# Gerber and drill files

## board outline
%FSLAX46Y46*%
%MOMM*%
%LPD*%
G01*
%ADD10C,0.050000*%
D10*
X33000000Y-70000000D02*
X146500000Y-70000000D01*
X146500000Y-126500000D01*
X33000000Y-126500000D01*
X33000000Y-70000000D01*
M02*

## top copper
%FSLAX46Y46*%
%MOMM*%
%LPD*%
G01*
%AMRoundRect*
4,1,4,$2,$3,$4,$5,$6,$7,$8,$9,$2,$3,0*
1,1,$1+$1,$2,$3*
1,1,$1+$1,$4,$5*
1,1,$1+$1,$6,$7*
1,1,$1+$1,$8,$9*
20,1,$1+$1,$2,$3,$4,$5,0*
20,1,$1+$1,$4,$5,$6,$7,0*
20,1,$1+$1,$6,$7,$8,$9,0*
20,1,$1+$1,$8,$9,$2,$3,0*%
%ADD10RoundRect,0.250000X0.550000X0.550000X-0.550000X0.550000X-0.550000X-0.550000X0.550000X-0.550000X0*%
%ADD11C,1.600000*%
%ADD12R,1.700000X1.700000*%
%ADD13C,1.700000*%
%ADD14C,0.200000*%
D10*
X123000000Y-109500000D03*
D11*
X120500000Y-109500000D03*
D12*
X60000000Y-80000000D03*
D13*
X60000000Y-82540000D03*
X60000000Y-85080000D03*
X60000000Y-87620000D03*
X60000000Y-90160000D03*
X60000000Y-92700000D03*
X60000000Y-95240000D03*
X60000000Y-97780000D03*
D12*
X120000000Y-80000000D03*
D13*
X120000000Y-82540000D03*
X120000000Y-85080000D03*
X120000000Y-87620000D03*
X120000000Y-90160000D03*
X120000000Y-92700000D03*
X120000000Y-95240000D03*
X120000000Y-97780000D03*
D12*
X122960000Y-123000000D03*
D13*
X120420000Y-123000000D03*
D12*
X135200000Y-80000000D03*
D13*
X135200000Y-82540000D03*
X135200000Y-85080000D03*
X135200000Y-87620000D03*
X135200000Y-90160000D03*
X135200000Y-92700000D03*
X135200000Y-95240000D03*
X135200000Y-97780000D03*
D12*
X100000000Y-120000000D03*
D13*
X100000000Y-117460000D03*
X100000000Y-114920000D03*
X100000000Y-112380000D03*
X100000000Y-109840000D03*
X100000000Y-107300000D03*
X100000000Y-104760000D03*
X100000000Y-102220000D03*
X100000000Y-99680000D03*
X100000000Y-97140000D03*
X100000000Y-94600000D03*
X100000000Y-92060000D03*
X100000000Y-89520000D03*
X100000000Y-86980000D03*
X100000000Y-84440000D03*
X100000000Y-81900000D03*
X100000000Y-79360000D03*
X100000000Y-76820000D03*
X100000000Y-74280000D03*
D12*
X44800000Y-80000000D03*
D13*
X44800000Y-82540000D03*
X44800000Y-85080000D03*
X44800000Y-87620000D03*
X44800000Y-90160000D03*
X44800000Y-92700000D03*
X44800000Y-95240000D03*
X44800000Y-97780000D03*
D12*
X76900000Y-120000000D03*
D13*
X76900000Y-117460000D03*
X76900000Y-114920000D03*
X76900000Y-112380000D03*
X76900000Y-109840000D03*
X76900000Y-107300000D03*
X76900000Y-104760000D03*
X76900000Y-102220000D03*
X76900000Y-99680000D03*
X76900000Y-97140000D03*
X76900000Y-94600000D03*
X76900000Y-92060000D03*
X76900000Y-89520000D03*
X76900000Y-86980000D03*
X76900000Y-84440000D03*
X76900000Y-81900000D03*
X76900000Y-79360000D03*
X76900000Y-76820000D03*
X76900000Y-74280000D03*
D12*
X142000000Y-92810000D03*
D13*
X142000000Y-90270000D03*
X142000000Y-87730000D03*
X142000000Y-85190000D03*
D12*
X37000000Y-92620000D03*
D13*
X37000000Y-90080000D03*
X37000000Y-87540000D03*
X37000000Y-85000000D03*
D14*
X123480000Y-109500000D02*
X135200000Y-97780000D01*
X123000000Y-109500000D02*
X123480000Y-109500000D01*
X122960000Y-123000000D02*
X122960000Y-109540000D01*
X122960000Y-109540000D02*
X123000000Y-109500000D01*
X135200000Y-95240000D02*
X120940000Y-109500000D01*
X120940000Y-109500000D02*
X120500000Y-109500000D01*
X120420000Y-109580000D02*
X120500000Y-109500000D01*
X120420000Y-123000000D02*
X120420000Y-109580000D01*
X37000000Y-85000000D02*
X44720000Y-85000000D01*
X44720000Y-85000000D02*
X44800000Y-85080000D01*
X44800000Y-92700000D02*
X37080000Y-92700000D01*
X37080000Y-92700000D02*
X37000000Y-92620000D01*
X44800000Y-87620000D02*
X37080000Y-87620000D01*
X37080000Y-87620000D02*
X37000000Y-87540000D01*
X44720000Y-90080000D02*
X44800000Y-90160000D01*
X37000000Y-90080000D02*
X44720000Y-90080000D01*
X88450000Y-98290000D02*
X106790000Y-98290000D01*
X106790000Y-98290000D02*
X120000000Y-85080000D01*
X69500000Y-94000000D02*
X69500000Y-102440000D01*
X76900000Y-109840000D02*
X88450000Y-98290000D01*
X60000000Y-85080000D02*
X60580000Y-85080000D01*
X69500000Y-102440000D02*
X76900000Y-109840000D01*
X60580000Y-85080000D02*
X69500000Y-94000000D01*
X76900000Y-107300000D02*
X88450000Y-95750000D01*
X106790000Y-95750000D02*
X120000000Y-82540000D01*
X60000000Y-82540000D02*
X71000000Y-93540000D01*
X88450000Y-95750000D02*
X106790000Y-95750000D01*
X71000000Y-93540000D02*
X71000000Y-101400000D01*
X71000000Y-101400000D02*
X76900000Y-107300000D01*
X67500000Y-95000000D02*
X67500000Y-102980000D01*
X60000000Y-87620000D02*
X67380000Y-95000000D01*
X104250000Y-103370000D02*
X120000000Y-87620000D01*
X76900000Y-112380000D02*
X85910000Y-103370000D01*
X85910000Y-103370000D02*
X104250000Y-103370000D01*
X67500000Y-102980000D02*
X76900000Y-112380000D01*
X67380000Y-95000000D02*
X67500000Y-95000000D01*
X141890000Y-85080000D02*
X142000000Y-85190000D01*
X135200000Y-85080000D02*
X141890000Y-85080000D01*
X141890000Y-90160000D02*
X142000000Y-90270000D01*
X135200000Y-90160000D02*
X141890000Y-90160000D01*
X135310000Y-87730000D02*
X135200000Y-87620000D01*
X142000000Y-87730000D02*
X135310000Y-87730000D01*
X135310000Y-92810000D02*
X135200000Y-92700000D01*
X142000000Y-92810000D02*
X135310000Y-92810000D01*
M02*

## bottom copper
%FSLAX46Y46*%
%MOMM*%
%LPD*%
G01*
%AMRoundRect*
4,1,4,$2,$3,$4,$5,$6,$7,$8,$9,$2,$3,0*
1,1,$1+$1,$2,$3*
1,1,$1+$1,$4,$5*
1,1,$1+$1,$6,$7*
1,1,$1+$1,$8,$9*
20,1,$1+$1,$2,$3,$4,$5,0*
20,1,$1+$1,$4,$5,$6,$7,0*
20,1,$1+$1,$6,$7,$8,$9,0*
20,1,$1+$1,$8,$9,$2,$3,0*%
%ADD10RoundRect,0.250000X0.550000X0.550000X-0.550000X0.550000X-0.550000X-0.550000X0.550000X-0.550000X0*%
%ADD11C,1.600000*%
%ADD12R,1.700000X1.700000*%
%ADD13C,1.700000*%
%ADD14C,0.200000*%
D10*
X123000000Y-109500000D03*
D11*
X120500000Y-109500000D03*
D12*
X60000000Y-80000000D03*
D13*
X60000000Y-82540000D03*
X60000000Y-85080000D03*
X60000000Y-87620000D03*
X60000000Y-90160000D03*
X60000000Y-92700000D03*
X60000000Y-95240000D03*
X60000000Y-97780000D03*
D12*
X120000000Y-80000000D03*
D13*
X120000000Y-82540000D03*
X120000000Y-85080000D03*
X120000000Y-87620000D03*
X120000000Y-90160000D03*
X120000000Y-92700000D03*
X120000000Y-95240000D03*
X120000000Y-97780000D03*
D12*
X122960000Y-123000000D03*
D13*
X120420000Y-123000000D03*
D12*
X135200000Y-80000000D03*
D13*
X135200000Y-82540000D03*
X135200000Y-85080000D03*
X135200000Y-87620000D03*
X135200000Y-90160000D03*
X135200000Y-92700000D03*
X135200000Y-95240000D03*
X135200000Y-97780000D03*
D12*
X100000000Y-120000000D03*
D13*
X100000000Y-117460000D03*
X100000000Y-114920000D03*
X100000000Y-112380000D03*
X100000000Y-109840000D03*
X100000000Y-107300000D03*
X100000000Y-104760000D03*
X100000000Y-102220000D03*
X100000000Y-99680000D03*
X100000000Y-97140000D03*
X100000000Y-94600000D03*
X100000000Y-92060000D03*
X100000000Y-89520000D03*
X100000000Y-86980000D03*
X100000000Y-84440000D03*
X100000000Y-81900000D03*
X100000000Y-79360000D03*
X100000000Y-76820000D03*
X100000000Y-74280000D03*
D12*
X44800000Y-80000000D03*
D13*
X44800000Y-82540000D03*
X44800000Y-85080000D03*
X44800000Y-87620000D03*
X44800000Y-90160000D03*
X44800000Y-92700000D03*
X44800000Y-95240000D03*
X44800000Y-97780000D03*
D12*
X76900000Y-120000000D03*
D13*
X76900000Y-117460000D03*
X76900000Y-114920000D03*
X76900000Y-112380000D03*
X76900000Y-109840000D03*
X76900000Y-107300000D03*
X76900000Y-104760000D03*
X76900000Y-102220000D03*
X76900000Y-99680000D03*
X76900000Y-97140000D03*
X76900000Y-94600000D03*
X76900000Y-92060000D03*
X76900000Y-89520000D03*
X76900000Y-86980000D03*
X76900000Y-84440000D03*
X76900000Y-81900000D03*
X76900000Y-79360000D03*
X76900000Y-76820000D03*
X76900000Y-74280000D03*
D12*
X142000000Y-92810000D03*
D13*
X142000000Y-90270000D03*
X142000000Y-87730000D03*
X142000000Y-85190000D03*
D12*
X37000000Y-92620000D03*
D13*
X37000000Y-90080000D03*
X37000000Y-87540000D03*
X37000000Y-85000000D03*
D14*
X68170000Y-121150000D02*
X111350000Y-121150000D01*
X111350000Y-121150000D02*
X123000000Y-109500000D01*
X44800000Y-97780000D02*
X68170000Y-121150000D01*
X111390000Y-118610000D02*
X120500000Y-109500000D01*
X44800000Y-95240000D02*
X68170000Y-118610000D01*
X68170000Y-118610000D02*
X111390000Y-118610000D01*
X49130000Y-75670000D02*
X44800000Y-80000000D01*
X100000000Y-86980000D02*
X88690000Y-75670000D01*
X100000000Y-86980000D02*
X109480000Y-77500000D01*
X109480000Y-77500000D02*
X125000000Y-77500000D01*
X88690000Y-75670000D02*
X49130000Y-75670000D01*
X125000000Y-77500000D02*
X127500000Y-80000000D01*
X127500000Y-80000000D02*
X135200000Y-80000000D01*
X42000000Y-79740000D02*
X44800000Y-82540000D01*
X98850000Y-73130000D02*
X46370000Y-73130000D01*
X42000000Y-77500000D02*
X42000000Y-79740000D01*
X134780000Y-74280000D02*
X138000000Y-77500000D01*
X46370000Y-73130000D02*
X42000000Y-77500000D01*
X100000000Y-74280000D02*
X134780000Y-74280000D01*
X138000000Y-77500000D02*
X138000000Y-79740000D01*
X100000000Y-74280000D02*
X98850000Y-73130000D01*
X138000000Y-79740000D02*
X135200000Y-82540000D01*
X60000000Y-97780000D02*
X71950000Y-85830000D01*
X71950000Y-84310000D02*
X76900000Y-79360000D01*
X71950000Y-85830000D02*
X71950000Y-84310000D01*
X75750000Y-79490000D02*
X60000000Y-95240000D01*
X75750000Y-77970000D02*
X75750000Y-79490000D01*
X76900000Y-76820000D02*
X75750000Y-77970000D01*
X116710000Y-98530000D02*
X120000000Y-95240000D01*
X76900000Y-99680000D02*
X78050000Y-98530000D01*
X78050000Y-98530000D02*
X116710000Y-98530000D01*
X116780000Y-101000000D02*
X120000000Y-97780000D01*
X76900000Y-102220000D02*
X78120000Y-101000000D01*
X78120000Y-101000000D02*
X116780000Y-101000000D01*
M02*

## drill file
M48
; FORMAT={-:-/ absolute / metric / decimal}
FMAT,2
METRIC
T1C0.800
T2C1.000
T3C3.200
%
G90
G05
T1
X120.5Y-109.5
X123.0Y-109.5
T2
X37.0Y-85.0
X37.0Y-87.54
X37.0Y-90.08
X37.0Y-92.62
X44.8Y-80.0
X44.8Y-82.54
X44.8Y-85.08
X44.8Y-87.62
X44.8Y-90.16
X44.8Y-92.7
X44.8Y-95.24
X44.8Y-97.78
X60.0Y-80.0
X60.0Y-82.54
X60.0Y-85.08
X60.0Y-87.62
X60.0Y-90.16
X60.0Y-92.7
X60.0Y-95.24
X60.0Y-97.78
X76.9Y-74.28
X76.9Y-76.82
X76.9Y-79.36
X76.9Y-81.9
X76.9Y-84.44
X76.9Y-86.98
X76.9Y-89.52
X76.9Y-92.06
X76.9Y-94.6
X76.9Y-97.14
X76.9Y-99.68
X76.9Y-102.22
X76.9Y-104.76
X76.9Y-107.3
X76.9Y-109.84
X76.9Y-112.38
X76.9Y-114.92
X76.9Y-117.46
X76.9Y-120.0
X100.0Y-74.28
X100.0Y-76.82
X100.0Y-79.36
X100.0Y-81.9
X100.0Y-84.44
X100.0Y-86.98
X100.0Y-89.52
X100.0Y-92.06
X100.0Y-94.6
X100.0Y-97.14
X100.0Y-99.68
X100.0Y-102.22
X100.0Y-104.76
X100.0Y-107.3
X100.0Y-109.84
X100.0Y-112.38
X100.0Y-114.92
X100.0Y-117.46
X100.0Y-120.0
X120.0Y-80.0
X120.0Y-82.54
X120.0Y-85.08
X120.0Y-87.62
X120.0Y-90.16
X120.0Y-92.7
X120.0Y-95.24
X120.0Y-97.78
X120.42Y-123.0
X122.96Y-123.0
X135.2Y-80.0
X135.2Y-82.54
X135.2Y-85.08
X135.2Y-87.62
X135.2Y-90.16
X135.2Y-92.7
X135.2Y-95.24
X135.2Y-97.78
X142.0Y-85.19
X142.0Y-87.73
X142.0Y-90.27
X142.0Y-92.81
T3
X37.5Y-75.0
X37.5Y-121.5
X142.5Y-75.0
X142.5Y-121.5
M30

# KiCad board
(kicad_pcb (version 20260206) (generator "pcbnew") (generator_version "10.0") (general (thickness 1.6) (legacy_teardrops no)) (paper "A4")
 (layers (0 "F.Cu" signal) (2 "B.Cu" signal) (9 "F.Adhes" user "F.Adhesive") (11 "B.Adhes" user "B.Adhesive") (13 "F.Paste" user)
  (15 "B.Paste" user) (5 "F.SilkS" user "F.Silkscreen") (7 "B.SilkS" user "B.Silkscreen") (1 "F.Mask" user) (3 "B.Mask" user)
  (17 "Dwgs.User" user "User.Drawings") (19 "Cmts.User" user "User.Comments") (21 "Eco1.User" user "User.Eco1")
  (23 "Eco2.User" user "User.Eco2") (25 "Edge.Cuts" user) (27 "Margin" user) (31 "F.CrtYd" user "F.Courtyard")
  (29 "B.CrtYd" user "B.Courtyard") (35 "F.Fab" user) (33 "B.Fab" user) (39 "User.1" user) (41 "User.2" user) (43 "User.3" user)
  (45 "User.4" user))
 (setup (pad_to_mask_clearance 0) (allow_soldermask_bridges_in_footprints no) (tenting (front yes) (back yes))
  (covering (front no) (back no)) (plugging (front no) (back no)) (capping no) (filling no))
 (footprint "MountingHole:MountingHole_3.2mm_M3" (layer "F.Cu") (at 37.5 121.5)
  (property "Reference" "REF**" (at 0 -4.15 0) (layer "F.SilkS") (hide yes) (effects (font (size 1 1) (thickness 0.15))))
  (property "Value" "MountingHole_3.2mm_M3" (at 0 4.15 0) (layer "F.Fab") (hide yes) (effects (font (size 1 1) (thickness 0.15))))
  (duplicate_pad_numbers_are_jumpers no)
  (pad "" np_thru_hole circle (at 0 0) (size 3.2 3.2) (drill 3.2) (layers "*.Cu" "*.Mask")))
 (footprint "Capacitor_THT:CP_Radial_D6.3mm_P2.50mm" (layer "F.Cu") (at 123 109.5 180)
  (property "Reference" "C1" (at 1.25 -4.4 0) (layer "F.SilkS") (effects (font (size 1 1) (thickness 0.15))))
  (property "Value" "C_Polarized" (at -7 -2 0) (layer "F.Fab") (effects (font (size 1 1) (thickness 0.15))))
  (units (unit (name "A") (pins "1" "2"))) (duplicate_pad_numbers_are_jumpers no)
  (pad "1" thru_hole roundrect (at 0 0 180) (size 1.6 1.6) (drill 0.8) (layers "*.Cu" "*.Mask") (remove_unused_layers no)
   (roundrect_rratio 0.15625) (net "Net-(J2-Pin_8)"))
  (pad "2" thru_hole circle (at 2.5 0 180) (size 1.6 1.6) (drill 0.8) (layers "*.Cu" "*.Mask") (remove_unused_layers no)
   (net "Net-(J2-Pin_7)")))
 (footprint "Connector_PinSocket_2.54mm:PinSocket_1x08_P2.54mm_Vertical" (layer "F.Cu") (at 60 80)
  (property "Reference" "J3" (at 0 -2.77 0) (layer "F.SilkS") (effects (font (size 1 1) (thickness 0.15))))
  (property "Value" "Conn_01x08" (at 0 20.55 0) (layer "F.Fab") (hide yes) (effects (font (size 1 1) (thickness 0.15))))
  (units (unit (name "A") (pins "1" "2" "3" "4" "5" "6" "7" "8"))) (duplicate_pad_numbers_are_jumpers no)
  (pad "1" thru_hole rect (at 0 0) (size 1.7 1.7) (drill 1) (layers "*.Cu" "*.Mask") (remove_unused_layers no)
   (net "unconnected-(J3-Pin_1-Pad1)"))
  (pad "2" thru_hole circle (at 0 2.54) (size 1.7 1.7) (drill 1) (layers "*.Cu" "*.Mask") (remove_unused_layers no) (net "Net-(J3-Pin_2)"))
  (pad "3" thru_hole circle (at 0 5.08) (size 1.7 1.7) (drill 1) (layers "*.Cu" "*.Mask") (remove_unused_layers no) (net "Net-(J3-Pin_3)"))
  (pad "4" thru_hole circle (at 0 7.62) (size 1.7 1.7) (drill 1) (layers "*.Cu" "*.Mask") (remove_unused_layers no) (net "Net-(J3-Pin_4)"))
  (pad "5" thru_hole circle (at 0 10.16) (size 1.7 1.7) (drill 1) (layers "*.Cu" "*.Mask") (remove_unused_layers no)
   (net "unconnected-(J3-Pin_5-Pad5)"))
  (pad "6" thru_hole circle (at 0 12.7) (size 1.7 1.7) (drill 1) (layers "*.Cu" "*.Mask") (remove_unused_layers no)
   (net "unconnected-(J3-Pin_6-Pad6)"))
  (pad "7" thru_hole circle (at 0 15.24) (size 1.7 1.7) (drill 1) (layers "*.Cu" "*.Mask") (remove_unused_layers no) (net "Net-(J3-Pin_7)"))
  (pad "8" thru_hole circle (at 0 17.78) (size 1.7 1.7) (drill 1) (layers "*.Cu" "*.Mask") (remove_unused_layers no) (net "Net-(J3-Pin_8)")))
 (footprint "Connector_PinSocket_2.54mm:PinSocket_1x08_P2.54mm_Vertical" (layer "F.Cu") (at 120 80)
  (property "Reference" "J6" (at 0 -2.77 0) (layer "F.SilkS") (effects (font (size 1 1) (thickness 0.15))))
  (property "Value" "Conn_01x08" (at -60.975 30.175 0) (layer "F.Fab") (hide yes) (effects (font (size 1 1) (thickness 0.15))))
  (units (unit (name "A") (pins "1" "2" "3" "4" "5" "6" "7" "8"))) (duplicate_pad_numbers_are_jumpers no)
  (pad "1" thru_hole rect (at 0 0) (size 1.7 1.7) (drill 1) (layers "*.Cu" "*.Mask") (remove_unused_layers no)
   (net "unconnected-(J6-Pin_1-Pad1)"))
  (pad "2" thru_hole circle (at 0 2.54) (size 1.7 1.7) (drill 1) (layers "*.Cu" "*.Mask") (remove_unused_layers no) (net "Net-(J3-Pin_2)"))
  (pad "3" thru_hole circle (at 0 5.08) (size 1.7 1.7) (drill 1) (layers "*.Cu" "*.Mask") (remove_unused_layers no) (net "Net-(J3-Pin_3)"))
  (pad "4" thru_hole circle (at 0 7.62) (size 1.7 1.7) (drill 1) (layers "*.Cu" "*.Mask") (remove_unused_layers no) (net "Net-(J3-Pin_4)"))
  (pad "5" thru_hole circle (at 0 10.16) (size 1.7 1.7) (drill 1) (layers "*.Cu" "*.Mask") (remove_unused_layers no)
   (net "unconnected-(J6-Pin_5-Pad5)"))
  (pad "6" thru_hole circle (at 0 12.7) (size 1.7 1.7) (drill 1) (layers "*.Cu" "*.Mask") (remove_unused_layers no)
   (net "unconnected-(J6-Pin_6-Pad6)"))
  (pad "7" thru_hole circle (at 0 15.24) (size 1.7 1.7) (drill 1) (layers "*.Cu" "*.Mask") (remove_unused_layers no) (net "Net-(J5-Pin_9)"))
  (pad "8" thru_hole circle (at 0 17.78) (size 1.7 1.7) (drill 1) (layers "*.Cu" "*.Mask") (remove_unused_layers no) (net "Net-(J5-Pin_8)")))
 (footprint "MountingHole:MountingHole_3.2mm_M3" (layer "F.Cu") (at 142.5 75)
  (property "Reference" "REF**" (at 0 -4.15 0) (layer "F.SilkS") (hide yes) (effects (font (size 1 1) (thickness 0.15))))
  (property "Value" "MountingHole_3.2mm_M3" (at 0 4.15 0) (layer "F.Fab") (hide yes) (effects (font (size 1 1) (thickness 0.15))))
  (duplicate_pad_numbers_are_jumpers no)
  (pad "" np_thru_hole circle (at 0 0) (size 3.2 3.2) (drill 3.2) (layers "*.Cu" "*.Mask")))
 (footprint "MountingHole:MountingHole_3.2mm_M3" (layer "F.Cu") (at 142.5 121.5)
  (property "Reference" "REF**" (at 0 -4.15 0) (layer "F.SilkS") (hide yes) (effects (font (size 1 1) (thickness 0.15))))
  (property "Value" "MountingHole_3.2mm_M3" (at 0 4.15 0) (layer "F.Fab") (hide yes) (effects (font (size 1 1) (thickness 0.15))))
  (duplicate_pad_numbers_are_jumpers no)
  (pad "" np_thru_hole circle (at 0 0) (size 3.2 3.2) (drill 3.2) (layers "*.Cu" "*.Mask")))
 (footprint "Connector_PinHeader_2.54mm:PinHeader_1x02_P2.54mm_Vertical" (layer "F.Cu") (at 122.96 123 -90)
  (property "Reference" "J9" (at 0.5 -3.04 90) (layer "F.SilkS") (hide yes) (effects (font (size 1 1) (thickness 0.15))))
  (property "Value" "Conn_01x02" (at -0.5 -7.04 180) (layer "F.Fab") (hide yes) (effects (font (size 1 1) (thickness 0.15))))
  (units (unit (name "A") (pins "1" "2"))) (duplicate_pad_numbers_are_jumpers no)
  (pad "1" thru_hole rect (at 0 0 270) (size 1.7 1.7) (drill 1) (layers "*.Cu" "*.Mask") (remove_unused_layers no) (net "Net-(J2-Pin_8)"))
  (pad "2" thru_hole circle (at 0 2.54 270) (size 1.7 1.7) (drill 1) (layers "*.Cu" "*.Mask") (remove_unused_layers no)
   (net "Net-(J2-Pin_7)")))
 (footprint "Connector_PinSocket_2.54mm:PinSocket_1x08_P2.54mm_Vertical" (layer "F.Cu") (at 135.2 80)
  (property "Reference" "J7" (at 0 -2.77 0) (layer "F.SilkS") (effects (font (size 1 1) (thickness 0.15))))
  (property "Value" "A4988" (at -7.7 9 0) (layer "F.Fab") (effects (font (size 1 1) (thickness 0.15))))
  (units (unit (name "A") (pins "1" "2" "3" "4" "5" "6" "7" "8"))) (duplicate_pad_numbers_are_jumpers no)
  (pad "1" thru_hole rect (at 0 0) (size 1.7 1.7) (drill 1) (layers "*.Cu" "*.Mask") (remove_unused_layers no) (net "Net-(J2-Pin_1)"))
  (pad "2" thru_hole circle (at 0 2.54) (size 1.7 1.7) (drill 1) (layers "*.Cu" "*.Mask") (remove_unused_layers no) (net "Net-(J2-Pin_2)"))
  (pad "3" thru_hole circle (at 0 5.08) (size 1.7 1.7) (drill 1) (layers "*.Cu" "*.Mask") (remove_unused_layers no) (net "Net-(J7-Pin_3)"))
  (pad "4" thru_hole circle (at 0 7.62) (size 1.7 1.7) (drill 1) (layers "*.Cu" "*.Mask") (remove_unused_layers no) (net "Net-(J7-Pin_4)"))
  (pad "5" thru_hole circle (at 0 10.16) (size 1.7 1.7) (drill 1) (layers "*.Cu" "*.Mask") (remove_unused_layers no) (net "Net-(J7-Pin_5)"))
  (pad "6" thru_hole circle (at 0 12.7) (size 1.7 1.7) (drill 1) (layers "*.Cu" "*.Mask") (remove_unused_layers no) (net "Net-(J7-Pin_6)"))
  (pad "7" thru_hole circle (at 0 15.24) (size 1.7 1.7) (drill 1) (layers "*.Cu" "*.Mask") (remove_unused_layers no) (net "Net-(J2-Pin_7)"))
  (pad "8" thru_hole circle (at 0 17.78) (size 1.7 1.7) (drill 1) (layers "*.Cu" "*.Mask") (remove_unused_layers no) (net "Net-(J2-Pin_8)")))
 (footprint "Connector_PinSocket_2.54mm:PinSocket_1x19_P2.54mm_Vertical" (layer "F.Cu") (at 100 120 180)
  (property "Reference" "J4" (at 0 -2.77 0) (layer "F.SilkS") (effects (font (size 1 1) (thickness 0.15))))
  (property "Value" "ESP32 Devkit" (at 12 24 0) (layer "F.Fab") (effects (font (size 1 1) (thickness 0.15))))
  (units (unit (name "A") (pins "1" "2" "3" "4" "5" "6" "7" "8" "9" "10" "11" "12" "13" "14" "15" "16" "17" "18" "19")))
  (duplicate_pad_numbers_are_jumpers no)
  (pad "1" thru_hole rect (at 0 0 180) (size 1.7 1.7) (drill 1) (layers "*.Cu" "*.Mask") (remove_unused_layers no)
   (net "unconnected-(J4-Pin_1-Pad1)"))
  (pad "2" thru_hole circle (at 0 2.54 180) (size 1.7 1.7) (drill 1) (layers "*.Cu" "*.Mask") (remove_unused_layers no)
   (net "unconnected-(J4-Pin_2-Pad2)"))
  (pad "3" thru_hole circle (at 0 5.08 180) (size 1.7 1.7) (drill 1) (layers "*.Cu" "*.Mask") (remove_unused_layers no)
   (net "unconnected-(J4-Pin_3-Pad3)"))
  (pad "4" thru_hole circle (at 0 7.62 180) (size 1.7 1.7) (drill 1) (layers "*.Cu" "*.Mask") (remove_unused_layers no)
   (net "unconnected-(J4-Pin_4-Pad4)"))
  (pad "5" thru_hole circle (at 0 10.16 180) (size 1.7 1.7) (drill 1) (layers "*.Cu" "*.Mask") (remove_unused_layers no)
   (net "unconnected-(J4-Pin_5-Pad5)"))
  (pad "6" thru_hole circle (at 0 12.7 180) (size 1.7 1.7) (drill 1) (layers "*.Cu" "*.Mask") (remove_unused_layers no)
   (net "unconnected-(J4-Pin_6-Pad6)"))
  (pad "7" thru_hole circle (at 0 15.24 180) (size 1.7 1.7) (drill 1) (layers "*.Cu" "*.Mask") (remove_unused_layers no)
   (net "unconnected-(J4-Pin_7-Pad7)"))
  (pad "8" thru_hole circle (at 0 17.78 180) (size 1.7 1.7) (drill 1) (layers "*.Cu" "*.Mask") (remove_unused_layers no)
   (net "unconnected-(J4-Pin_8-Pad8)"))
  (pad "9" thru_hole circle (at 0 20.32 180) (size 1.7 1.7) (drill 1) (layers "*.Cu" "*.Mask") (remove_unused_layers no)
   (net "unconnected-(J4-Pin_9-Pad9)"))
  (pad "10" thru_hole circle (at 0 22.86 180) (size 1.7 1.7) (drill 1) (layers "*.Cu" "*.Mask") (remove_unused_layers no)
   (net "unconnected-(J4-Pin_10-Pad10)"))
  (pad "11" thru_hole circle (at 0 25.4 180) (size 1.7 1.7) (drill 1) (layers "*.Cu" "*.Mask") (remove_unused_layers no)
   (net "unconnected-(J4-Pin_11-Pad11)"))
  (pad "12" thru_hole circle (at 0 27.94 180) (size 1.7 1.7) (drill 1) (layers "*.Cu" "*.Mask") (remove_unused_layers no)
   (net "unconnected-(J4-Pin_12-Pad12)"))
  (pad "13" thru_hole circle (at 0 30.48 180) (size 1.7 1.7) (drill 1) (layers "*.Cu" "*.Mask") (remove_unused_layers no)
   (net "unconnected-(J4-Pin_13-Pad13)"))
  (pad "14" thru_hole circle (at 0 33.02 180) (size 1.7 1.7) (drill 1) (layers "*.Cu" "*.Mask") (remove_unused_layers no)
   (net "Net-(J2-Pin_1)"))
  (pad "15" thru_hole circle (at 0 35.56 180) (size 1.7 1.7) (drill 1) (layers "*.Cu" "*.Mask") (remove_unused_layers no)
   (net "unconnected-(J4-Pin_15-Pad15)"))
  (pad "16" thru_hole circle (at 0 38.1 180) (size 1.7 1.7) (drill 1) (layers "*.Cu" "*.Mask") (remove_unused_layers no)
   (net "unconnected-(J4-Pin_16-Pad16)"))
  (pad "17" thru_hole circle (at 0 40.64 180) (size 1.7 1.7) (drill 1) (layers "*.Cu" "*.Mask") (remove_unused_layers no)
   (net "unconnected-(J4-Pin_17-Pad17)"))
  (pad "18" thru_hole circle (at 0 43.18 180) (size 1.7 1.7) (drill 1) (layers "*.Cu" "*.Mask") (remove_unused_layers no)
   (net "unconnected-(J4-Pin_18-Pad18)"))
  (pad "19" thru_hole circle (at 0 45.72 180) (size 1.7 1.7) (drill 1) (layers "*.Cu" "*.Mask") (remove_unused_layers no)
   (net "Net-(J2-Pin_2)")))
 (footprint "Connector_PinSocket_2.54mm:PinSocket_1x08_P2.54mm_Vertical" (layer "F.Cu") (at 44.8 80)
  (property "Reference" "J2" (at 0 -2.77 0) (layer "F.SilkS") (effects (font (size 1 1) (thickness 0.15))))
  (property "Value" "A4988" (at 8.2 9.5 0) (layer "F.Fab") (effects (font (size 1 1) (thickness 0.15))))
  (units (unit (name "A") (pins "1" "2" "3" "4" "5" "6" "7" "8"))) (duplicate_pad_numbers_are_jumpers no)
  (pad "1" thru_hole rect (at 0 0) (size 1.7 1.7) (drill 1) (layers "*.Cu" "*.Mask") (remove_unused_layers no) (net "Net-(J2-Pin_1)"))
  (pad "2" thru_hole circle (at 0 2.54) (size 1.7 1.7) (drill 1) (layers "*.Cu" "*.Mask") (remove_unused_layers no) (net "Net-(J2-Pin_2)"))
  (pad "3" thru_hole circle (at 0 5.08) (size 1.7 1.7) (drill 1) (layers "*.Cu" "*.Mask") (remove_unused_layers no) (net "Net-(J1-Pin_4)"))
  (pad "4" thru_hole circle (at 0 7.62) (size 1.7 1.7) (drill 1) (layers "*.Cu" "*.Mask") (remove_unused_layers no) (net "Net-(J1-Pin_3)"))
  (pad "5" thru_hole circle (at 0 10.16) (size 1.7 1.7) (drill 1) (layers "*.Cu" "*.Mask") (remove_unused_layers no) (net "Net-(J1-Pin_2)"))
  (pad "6" thru_hole circle (at 0 12.7) (size 1.7 1.7) (drill 1) (layers "*.Cu" "*.Mask") (remove_unused_layers no) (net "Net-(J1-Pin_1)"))
  (pad "7" thru_hole circle (at 0 15.24) (size 1.7 1.7) (drill 1) (layers "*.Cu" "*.Mask") (remove_unused_layers no) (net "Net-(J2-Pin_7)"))
  (pad "8" thru_hole circle (at 0 17.78) (size 1.7 1.7) (drill 1) (layers "*.Cu" "*.Mask") (remove_unused_layers no) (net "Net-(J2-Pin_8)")))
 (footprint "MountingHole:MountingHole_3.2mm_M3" (layer "F.Cu") (at 37.5 75)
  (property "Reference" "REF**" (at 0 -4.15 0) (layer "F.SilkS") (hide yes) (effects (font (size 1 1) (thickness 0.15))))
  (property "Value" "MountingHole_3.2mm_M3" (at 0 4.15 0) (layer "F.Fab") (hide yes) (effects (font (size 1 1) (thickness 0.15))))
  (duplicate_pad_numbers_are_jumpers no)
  (pad "" np_thru_hole circle (at 0 0) (size 3.2 3.2) (drill 3.2) (layers "*.Cu" "*.Mask")))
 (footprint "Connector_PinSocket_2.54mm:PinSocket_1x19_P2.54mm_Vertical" (layer "F.Cu") (at 76.9 120 180)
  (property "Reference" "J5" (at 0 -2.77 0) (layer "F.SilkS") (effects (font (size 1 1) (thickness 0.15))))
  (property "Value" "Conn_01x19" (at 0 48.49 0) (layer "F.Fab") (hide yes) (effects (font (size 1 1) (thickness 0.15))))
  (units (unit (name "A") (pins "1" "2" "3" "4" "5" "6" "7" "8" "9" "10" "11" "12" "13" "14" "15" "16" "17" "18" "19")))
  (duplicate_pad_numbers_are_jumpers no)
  (pad "1" thru_hole rect (at 0 0 180) (size 1.7 1.7) (drill 1) (layers "*.Cu" "*.Mask") (remove_unused_layers no)
   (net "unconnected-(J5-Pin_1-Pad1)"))
  (pad "2" thru_hole circle (at 0 2.54 180) (size 1.7 1.7) (drill 1) (layers "*.Cu" "*.Mask") (remove_unused_layers no)
   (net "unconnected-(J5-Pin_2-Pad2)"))
  (pad "3" thru_hole circle (at 0 5.08 180) (size 1.7 1.7) (drill 1) (layers "*.Cu" "*.Mask") (remove_unused_layers no)
   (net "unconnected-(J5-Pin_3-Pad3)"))
  (pad "4" thru_hole circle (at 0 7.62 180) (size 1.7 1.7) (drill 1) (layers "*.Cu" "*.Mask") (remove_unused_layers no)
   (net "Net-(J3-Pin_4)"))
  (pad "5" thru_hole circle (at 0 10.16 180) (size 1.7 1.7) (drill 1) (layers "*.Cu" "*.Mask") (remove_unused_layers no)
   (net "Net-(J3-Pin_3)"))
  (pad "6" thru_hole circle (at 0 12.7 180) (size 1.7 1.7) (drill 1) (layers "*.Cu" "*.Mask") (remove_unused_layers no)
   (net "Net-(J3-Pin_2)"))
  (pad "7" thru_hole circle (at 0 15.24 180) (size 1.7 1.7) (drill 1) (layers "*.Cu" "*.Mask") (remove_unused_layers no)
   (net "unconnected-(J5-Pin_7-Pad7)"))
  (pad "8" thru_hole circle (at 0 17.78 180) (size 1.7 1.7) (drill 1) (layers "*.Cu" "*.Mask") (remove_unused_layers no)
   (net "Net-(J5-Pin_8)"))
  (pad "9" thru_hole circle (at 0 20.32 180) (size 1.7 1.7) (drill 1) (layers "*.Cu" "*.Mask") (remove_unused_layers no)
   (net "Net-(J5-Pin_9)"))
  (pad "10" thru_hole circle (at 0 22.86 180) (size 1.7 1.7) (drill 1) (layers "*.Cu" "*.Mask") (remove_unused_layers no)
   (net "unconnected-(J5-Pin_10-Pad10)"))
  (pad "11" thru_hole circle (at 0 25.4 180) (size 1.7 1.7) (drill 1) (layers "*.Cu" "*.Mask") (remove_unused_layers no)
   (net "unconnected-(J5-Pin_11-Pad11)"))
  (pad "12" thru_hole circle (at 0 27.94 180) (size 1.7 1.7) (drill 1) (layers "*.Cu" "*.Mask") (remove_unused_layers no)
   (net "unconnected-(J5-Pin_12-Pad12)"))
  (pad "13" thru_hole circle (at 0 30.48 180) (size 1.7 1.7) (drill 1) (layers "*.Cu" "*.Mask") (remove_unused_layers no)
   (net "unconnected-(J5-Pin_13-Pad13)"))
  (pad "14" thru_hole circle (at 0 33.02 180) (size 1.7 1.7) (drill 1) (layers "*.Cu" "*.Mask") (remove_unused_layers no)
   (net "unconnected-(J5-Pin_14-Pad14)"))
  (pad "15" thru_hole circle (at 0 35.56 180) (size 1.7 1.7) (drill 1) (layers "*.Cu" "*.Mask") (remove_unused_layers no)
   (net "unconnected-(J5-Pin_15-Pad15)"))
  (pad "16" thru_hole circle (at 0 38.1 180) (size 1.7 1.7) (drill 1) (layers "*.Cu" "*.Mask") (remove_unused_layers no)
   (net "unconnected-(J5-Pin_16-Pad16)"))
  (pad "17" thru_hole circle (at 0 40.64 180) (size 1.7 1.7) (drill 1) (layers "*.Cu" "*.Mask") (remove_unused_layers no)
   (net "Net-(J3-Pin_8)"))
  (pad "18" thru_hole circle (at 0 43.18 180) (size 1.7 1.7) (drill 1) (layers "*.Cu" "*.Mask") (remove_unused_layers no)
   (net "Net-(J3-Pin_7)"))
  (pad "19" thru_hole circle (at 0 45.72 180) (size 1.7 1.7) (drill 1) (layers "*.Cu" "*.Mask") (remove_unused_layers no)
   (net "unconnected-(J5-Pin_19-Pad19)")))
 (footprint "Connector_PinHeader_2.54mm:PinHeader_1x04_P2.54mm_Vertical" (layer "F.Cu") (at 142 92.81 180)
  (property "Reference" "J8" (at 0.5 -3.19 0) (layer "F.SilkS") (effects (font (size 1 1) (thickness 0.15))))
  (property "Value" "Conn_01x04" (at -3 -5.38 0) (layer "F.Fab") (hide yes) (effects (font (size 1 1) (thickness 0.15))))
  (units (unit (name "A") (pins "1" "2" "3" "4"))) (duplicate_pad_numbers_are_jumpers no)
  (pad "1" thru_hole rect (at 0 0 180) (size 1.7 1.7) (drill 1) (layers "*.Cu" "*.Mask") (remove_unused_layers no) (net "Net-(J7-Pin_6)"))
  (pad "2" thru_hole circle (at 0 2.54 180) (size 1.7 1.7) (drill 1) (layers "*.Cu" "*.Mask") (remove_unused_layers no)
   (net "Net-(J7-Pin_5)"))
  (pad "3" thru_hole circle (at 0 5.08 180) (size 1.7 1.7) (drill 1) (layers "*.Cu" "*.Mask") (remove_unused_layers no)
   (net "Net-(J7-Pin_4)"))
  (pad "4" thru_hole circle (at 0 7.62 180) (size 1.7 1.7) (drill 1) (layers "*.Cu" "*.Mask") (remove_unused_layers no)
   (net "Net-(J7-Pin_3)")))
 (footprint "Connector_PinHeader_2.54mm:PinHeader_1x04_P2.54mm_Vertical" (layer "F.Cu") (at 37 92.62 180)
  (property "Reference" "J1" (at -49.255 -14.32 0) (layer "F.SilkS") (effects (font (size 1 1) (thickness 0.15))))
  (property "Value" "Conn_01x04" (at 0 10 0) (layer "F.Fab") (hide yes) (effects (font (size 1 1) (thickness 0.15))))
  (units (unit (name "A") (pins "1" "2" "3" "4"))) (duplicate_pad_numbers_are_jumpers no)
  (pad "1" thru_hole rect (at 0 0 180) (size 1.7 1.7) (drill 1) (layers "*.Cu" "*.Mask") (remove_unused_layers no) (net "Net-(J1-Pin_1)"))
  (pad "2" thru_hole circle (at 0 2.54 180) (size 1.7 1.7) (drill 1) (layers "*.Cu" "*.Mask") (remove_unused_layers no)
   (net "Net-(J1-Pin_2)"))
  (pad "3" thru_hole circle (at 0 5.08 180) (size 1.7 1.7) (drill 1) (layers "*.Cu" "*.Mask") (remove_unused_layers no)
   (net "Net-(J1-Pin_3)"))
  (pad "4" thru_hole circle (at 0 7.62 180) (size 1.7 1.7) (drill 1) (layers "*.Cu" "*.Mask") (remove_unused_layers no)
   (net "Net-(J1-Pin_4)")))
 (gr_rect (start 33 70) (end 146.5 126.5) (stroke (width 0.05) (type default)) (fill no) (layer "Edge.Cuts"))
 (segment (start 123.48 109.5) (end 135.2 97.78) (width 0.2) (layer "F.Cu") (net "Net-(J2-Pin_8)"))
 (segment (start 123 109.5) (end 123.48 109.5) (width 0.2) (layer "F.Cu") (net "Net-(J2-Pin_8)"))
 (segment (start 122.96 123) (end 122.96 109.54) (width 0.2) (layer "F.Cu") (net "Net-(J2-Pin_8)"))
 (segment (start 122.96 109.54) (end 123 109.5) (width 0.2) (layer "F.Cu") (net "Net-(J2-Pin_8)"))
 (segment (start 68.17 121.15) (end 111.35 121.15) (width 0.2) (layer "B.Cu") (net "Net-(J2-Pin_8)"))
 (segment (start 111.35 121.15) (end 123 109.5) (width 0.2) (layer "B.Cu") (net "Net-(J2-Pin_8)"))
 (segment (start 44.8 97.78) (end 68.17 121.15) (width 0.2) (layer "B.Cu") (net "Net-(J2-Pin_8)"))
 (segment (start 135.2 95.24) (end 120.94 109.5) (width 0.2) (layer "F.Cu") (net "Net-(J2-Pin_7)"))
 (segment (start 120.94 109.5) (end 120.5 109.5) (width 0.2) (layer "F.Cu") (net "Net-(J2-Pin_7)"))
 (segment (start 120.42 109.58) (end 120.5 109.5) (width 0.2) (layer "F.Cu") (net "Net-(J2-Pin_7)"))
 (segment (start 120.42 123) (end 120.42 109.58) (width 0.2) (layer "F.Cu") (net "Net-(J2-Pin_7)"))
 (segment (start 111.39 118.61) (end 120.5 109.5) (width 0.2) (layer "B.Cu") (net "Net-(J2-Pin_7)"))
 (segment (start 44.8 95.24) (end 68.17 118.61) (width 0.2) (layer "B.Cu") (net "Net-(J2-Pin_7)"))
 (segment (start 68.17 118.61) (end 111.39 118.61) (width 0.2) (layer "B.Cu") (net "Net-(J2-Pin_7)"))
 (segment (start 37 85) (end 44.72 85) (width 0.2) (layer "F.Cu") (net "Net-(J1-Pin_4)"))
 (segment (start 44.72 85) (end 44.8 85.08) (width 0.2) (layer "F.Cu") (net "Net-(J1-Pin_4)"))
 (segment (start 44.8 92.7) (end 37.08 92.7) (width 0.2) (layer "F.Cu") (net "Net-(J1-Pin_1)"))
 (segment (start 37.08 92.7) (end 37 92.62) (width 0.2) (layer "F.Cu") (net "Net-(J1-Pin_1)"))
 (segment (start 44.8 87.62) (end 37.08 87.62) (width 0.2) (layer "F.Cu") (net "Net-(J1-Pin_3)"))
 (segment (start 37.08 87.62) (end 37 87.54) (width 0.2) (layer "F.Cu") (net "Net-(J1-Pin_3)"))
 (segment (start 44.72 90.08) (end 44.8 90.16) (width 0.2) (layer "F.Cu") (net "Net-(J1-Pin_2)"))
 (segment (start 37 90.08) (end 44.72 90.08) (width 0.2) (layer "F.Cu") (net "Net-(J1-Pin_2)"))
 (segment (start 49.13 75.67) (end 44.8 80) (width 0.2) (layer "B.Cu") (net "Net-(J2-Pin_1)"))
 (segment (start 100 86.98) (end 88.69 75.67) (width 0.2) (layer "B.Cu") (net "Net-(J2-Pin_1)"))
 (segment (start 100 86.98) (end 109.48 77.5) (width 0.2) (layer "B.Cu") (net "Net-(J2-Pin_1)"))
 (segment (start 109.48 77.5) (end 125 77.5) (width 0.2) (layer "B.Cu") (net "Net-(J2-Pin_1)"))
 (segment (start 88.69 75.67) (end 49.13 75.67) (width 0.2) (layer "B.Cu") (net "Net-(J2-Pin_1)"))
 (segment (start 125 77.5) (end 127.5 80) (width 0.2) (layer "B.Cu") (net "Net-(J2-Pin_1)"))
 (segment (start 127.5 80) (end 135.2 80) (width 0.2) (layer "B.Cu") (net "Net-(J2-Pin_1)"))
 (segment (start 42 79.74) (end 44.8 82.54) (width 0.2) (layer "B.Cu") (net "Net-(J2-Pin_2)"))
 (segment (start 98.85 73.13) (end 46.37 73.13) (width 0.2) (layer "B.Cu") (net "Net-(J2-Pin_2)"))
 (segment (start 42 77.5) (end 42 79.74) (width 0.2) (layer "B.Cu") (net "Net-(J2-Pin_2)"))
 (segment (start 134.78 74.28) (end 138 77.5) (width 0.2) (layer "B.Cu") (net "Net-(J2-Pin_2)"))
 (segment (start 46.37 73.13) (end 42 77.5) (width 0.2) (layer "B.Cu") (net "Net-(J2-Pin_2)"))
 (segment (start 100 74.28) (end 134.78 74.28) (width 0.2) (layer "B.Cu") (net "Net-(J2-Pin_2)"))
 (segment (start 138 77.5) (end 138 79.74) (width 0.2) (layer "B.Cu") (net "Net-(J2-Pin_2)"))
 (segment (start 100 74.28) (end 98.85 73.13) (width 0.2) (layer "B.Cu") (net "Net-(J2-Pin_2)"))
 (segment (start 138 79.74) (end 135.2 82.54) (width 0.2) (layer "B.Cu") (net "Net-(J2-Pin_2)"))
 (segment (start 60 97.78) (end 71.95 85.83) (width 0.2) (layer "B.Cu") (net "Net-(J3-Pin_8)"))
 (segment (start 71.95 84.31) (end 76.9 79.36) (width 0.2) (layer "B.Cu") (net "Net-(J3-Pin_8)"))
 (segment (start 71.95 85.83) (end 71.95 84.31) (width 0.2) (layer "B.Cu") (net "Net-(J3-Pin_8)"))
 (segment (start 75.75 79.49) (end 60 95.24) (width 0.2) (layer "B.Cu") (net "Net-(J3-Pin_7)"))
 (segment (start 75.75 77.97) (end 75.75 79.49) (width 0.2) (layer "B.Cu") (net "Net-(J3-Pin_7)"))
 (segment (start 76.9 76.82) (end 75.75 77.97) (width 0.2) (layer "B.Cu") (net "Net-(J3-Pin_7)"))
 (segment (start 88.45 98.29) (end 106.79 98.29) (width 0.2) (layer "F.Cu") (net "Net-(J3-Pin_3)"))
 (segment (start 106.79 98.29) (end 120 85.08) (width 0.2) (layer "F.Cu") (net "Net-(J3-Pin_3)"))
 (segment (start 69.5 94) (end 69.5 102.44) (width 0.2) (layer "F.Cu") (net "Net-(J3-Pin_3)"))
 (segment (start 76.9 109.84) (end 88.45 98.29) (width 0.2) (layer "F.Cu") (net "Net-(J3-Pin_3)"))
 (segment (start 60 85.08) (end 60.58 85.08) (width 0.2) (layer "F.Cu") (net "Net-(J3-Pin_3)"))
 (segment (start 69.5 102.44) (end 76.9 109.84) (width 0.2) (layer "F.Cu") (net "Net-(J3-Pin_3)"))
 (segment (start 60.58 85.08) (end 69.5 94) (width 0.2) (layer "F.Cu") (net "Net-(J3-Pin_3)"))
 (segment (start 76.9 107.3) (end 88.45 95.75) (width 0.2) (layer "F.Cu") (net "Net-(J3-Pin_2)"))
 (segment (start 106.79 95.75) (end 120 82.54) (width 0.2) (layer "F.Cu") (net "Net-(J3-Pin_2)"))
 (segment (start 60 82.54) (end 71 93.54) (width 0.2) (layer "F.Cu") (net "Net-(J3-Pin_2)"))
 (segment (start 88.45 95.75) (end 106.79 95.75) (width 0.2) (layer "F.Cu") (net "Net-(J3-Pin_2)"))
 (segment (start 71 93.54) (end 71 101.4) (width 0.2) (layer "F.Cu") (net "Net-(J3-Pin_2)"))
 (segment (start 71 101.4) (end 76.9 107.3) (width 0.2) (layer "F.Cu") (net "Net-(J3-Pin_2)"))
 (segment (start 67.5 95) (end 67.5 102.98) (width 0.2) (layer "F.Cu") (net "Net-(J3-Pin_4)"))
 (segment (start 60 87.62) (end 67.38 95) (width 0.2) (layer "F.Cu") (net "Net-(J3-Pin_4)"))
 (segment (start 104.25 103.37) (end 120 87.62) (width 0.2) (layer "F.Cu") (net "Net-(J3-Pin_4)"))
 (segment (start 76.9 112.38) (end 85.91 103.37) (width 0.2) (layer "F.Cu") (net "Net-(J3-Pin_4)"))
 (segment (start 85.91 103.37) (end 104.25 103.37) (width 0.2) (layer "F.Cu") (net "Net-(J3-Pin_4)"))
 (segment (start 67.5 102.98) (end 76.9 112.38) (width 0.2) (layer "F.Cu") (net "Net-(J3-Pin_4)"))
 (segment (start 67.38 95) (end 67.5 95) (width 0.2) (layer "F.Cu") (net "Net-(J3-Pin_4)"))
 (segment (start 116.71 98.53) (end 120 95.24) (width 0.2) (layer "B.Cu") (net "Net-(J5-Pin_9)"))
 (segment (start 76.9 99.68) (end 78.05 98.53) (width 0.2) (layer "B.Cu") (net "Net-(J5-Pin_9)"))
 (segment (start 78.05 98.53) (end 116.71 98.53) (width 0.2) (layer "B.Cu") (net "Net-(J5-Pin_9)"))
 (segment (start 116.78 101) (end 120 97.78) (width 0.2) (layer "B.Cu") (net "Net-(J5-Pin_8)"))
 (segment (start 76.9 102.22) (end 78.12 101) (width 0.2) (layer "B.Cu") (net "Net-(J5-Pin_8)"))
 (segment (start 78.12 101) (end 116.78 101) (width 0.2) (layer "B.Cu") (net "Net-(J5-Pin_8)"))
 (segment (start 141.89 85.08) (end 142 85.19) (width 0.2) (layer "F.Cu") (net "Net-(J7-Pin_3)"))
 (segment (start 135.2 85.08) (end 141.89 85.08) (width 0.2) (layer "F.Cu") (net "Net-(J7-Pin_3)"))
 (segment (start 141.89 90.16) (end 142 90.27) (width 0.2) (layer "F.Cu") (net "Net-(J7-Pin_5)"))
 (segment (start 135.2 90.16) (end 141.89 90.16) (width 0.2) (layer "F.Cu") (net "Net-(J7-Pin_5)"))
 (segment (start 135.31 87.73) (end 135.2 87.62) (width 0.2) (layer "F.Cu") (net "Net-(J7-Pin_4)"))
 (segment (start 142 87.73) (end 135.31 87.73) (width 0.2) (layer "F.Cu") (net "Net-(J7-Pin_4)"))
 (segment (start 135.31 92.81) (end 135.2 92.7) (width 0.2) (layer "F.Cu") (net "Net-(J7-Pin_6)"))
 (segment (start 142 92.81) (end 135.31 92.81) (width 0.2) (layer "F.Cu") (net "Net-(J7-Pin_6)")))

